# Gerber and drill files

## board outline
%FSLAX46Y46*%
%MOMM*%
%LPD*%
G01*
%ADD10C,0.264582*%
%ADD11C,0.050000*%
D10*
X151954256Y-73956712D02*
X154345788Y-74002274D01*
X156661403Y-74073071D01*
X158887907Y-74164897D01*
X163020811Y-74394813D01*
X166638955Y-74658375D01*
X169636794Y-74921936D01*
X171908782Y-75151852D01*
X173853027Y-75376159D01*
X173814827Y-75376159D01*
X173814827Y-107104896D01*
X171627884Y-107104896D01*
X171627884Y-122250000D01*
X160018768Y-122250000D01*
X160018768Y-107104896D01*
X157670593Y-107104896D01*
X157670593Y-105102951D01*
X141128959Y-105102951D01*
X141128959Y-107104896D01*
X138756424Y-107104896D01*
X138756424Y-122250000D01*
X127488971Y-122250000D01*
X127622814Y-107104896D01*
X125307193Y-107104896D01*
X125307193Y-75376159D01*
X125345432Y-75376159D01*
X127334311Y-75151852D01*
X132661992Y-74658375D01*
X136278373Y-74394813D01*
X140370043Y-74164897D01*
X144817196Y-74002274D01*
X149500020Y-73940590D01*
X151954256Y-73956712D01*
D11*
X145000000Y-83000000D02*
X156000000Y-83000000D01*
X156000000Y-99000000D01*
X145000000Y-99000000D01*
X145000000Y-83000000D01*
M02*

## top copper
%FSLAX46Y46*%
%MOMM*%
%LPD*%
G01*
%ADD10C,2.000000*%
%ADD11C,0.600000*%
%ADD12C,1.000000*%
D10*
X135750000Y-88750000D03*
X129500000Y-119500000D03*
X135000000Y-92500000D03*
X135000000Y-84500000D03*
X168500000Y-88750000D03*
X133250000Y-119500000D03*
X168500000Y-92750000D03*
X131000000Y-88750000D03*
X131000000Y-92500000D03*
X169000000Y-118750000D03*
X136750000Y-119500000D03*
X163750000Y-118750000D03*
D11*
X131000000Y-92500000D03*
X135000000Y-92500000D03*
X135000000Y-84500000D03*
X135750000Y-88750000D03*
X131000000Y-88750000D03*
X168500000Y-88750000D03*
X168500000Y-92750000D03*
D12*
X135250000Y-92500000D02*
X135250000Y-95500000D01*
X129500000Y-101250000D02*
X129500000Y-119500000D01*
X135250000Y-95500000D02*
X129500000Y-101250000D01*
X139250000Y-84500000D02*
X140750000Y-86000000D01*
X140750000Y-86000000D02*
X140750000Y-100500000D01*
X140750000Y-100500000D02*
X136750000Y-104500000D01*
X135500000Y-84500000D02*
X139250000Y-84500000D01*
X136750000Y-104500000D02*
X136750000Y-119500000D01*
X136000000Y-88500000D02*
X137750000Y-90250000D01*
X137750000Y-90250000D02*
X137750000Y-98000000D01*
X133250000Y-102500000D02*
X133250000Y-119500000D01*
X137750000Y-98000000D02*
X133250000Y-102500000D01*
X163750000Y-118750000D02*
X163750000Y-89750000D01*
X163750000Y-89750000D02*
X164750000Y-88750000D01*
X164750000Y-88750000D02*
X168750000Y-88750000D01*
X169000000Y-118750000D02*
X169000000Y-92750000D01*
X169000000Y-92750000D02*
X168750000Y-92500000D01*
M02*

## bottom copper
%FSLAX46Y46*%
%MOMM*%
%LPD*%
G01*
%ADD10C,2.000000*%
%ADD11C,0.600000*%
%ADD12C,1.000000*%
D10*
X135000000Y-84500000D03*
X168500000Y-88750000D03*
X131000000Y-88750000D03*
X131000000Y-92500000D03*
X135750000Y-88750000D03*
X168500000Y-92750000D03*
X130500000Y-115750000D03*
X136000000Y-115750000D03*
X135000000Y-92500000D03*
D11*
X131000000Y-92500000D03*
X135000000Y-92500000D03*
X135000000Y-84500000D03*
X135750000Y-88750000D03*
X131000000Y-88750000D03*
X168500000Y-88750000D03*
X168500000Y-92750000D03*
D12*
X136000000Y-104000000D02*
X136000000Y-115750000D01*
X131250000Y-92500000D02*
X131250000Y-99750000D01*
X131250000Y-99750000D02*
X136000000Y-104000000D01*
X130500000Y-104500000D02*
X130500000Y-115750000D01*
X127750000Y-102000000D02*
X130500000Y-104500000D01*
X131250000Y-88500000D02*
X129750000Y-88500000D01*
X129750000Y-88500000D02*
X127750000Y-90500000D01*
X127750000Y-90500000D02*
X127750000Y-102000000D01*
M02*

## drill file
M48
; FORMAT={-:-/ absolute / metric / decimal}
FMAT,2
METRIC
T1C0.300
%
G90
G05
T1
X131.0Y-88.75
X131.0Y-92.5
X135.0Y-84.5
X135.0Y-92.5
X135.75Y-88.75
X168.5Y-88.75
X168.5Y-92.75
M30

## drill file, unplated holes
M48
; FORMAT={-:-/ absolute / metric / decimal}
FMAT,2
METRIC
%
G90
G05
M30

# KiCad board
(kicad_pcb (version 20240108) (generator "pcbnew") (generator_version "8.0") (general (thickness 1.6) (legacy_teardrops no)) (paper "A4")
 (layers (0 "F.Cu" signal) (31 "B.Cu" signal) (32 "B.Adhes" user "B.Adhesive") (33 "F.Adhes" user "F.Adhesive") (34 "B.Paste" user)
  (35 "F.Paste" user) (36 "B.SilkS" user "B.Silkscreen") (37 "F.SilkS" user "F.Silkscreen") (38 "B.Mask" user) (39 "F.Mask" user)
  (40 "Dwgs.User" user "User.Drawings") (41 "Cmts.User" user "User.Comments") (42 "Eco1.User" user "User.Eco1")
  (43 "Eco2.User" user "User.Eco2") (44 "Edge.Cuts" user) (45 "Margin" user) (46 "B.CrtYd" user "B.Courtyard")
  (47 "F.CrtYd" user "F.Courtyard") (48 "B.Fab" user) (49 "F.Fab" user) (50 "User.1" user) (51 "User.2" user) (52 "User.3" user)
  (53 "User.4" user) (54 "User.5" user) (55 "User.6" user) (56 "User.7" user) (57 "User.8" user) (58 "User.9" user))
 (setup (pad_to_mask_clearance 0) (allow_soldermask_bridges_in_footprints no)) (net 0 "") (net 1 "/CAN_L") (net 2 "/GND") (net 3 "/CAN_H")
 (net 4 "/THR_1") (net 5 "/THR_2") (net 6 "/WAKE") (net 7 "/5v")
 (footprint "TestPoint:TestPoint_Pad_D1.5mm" (layer "F.Cu") (at 135.75 88.75)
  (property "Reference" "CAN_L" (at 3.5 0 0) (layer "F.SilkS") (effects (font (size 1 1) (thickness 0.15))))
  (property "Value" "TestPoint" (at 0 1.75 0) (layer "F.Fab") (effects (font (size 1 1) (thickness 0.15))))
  (pad "1" smd circle (at 0 0) (size 2 2) (layers "F.Cu" "F.Mask") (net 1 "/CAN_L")))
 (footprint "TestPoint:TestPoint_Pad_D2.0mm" (layer "F.Cu") (at 129.5 119.5)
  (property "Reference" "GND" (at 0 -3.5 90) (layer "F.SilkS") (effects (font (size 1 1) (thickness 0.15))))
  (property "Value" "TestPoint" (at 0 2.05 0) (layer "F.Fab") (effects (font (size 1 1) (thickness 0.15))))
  (pad "1" smd circle (at 0 0) (size 2 2) (layers "F.Cu" "F.Mask") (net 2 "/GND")))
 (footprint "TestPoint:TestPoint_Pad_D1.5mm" (layer "F.Cu") (at 135 92.5)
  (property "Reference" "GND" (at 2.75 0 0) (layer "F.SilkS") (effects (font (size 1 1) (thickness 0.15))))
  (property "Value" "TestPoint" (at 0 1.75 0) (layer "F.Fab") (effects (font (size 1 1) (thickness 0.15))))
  (pad "1" smd circle (at 0 0) (size 2 2) (layers "F.Cu" "F.Mask") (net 2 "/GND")))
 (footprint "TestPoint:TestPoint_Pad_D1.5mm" (layer "F.Cu") (at 135 84.5)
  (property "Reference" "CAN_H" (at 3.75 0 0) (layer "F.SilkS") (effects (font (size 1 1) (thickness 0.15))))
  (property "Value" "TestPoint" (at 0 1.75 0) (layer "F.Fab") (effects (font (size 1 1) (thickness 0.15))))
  (pad "1" smd circle (at 0 0) (size 2 2) (layers "F.Cu" "F.Mask") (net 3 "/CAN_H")))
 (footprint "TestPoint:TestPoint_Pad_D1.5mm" (layer "F.Cu") (at 168.5 88.75)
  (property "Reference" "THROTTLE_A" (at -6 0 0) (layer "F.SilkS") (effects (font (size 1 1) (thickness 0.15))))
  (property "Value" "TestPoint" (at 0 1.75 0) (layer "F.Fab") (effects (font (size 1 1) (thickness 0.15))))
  (pad "1" smd circle (at 0 0) (size 2 2) (layers "F.Cu" "F.Mask") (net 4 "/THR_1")))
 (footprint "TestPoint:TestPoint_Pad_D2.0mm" (layer "F.Cu") (at 133.25 119.5)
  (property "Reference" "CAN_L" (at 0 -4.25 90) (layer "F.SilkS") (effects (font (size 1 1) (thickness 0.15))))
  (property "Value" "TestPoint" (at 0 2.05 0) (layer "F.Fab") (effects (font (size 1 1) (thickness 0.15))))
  (pad "1" smd circle (at 0 0) (size 2 2) (layers "F.Cu" "F.Mask") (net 1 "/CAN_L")))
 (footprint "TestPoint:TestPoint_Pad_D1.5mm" (layer "F.Cu") (at 168.5 92.75)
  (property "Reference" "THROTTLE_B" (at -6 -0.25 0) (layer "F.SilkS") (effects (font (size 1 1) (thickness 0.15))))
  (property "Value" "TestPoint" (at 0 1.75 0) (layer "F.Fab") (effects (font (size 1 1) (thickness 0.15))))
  (pad "1" smd circle (at 0 0) (size 2 2) (layers "F.Cu" "F.Mask") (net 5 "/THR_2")))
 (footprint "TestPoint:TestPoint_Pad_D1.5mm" (layer "F.Cu") (at 131 88.75)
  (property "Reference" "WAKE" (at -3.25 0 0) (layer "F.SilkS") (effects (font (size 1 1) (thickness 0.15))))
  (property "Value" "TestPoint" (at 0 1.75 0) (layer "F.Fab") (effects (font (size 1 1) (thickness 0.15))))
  (pad "1" smd circle (at 0 0) (size 2 2) (layers "F.Cu" "F.Mask") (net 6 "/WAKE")))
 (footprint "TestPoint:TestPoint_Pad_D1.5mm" (layer "F.Cu") (at 131 92.5)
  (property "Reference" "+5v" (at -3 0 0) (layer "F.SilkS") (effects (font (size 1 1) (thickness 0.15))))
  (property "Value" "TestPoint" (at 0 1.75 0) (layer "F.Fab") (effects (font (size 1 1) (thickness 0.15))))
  (pad "1" smd circle (at 0 0) (size 2 2) (layers "F.Cu" "F.Mask") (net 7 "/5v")))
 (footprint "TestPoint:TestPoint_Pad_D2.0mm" (layer "F.Cu") (at 169 118.75)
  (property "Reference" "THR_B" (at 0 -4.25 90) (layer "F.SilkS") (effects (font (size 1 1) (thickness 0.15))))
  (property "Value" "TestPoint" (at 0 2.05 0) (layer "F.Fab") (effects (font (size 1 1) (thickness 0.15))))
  (pad "1" smd circle (at 0 0) (size 2 2) (layers "F.Cu" "F.Mask") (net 5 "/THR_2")))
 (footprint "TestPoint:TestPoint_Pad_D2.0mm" (layer "F.Cu") (at 136.75 119.5)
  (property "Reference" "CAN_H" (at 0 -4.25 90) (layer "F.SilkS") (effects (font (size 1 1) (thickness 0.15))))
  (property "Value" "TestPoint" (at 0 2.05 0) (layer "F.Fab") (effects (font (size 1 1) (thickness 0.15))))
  (pad "1" smd circle (at 0 0) (size 2 2) (layers "F.Cu" "F.Mask") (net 3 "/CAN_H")))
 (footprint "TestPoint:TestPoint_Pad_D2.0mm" (layer "F.Cu") (at 163.75 118.75)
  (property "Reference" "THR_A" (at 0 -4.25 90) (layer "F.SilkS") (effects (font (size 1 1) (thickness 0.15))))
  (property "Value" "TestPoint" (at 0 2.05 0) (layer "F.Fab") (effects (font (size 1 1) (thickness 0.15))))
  (pad "1" smd circle (at 0 0) (size 2 2) (layers "F.Cu" "F.Mask") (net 4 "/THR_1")))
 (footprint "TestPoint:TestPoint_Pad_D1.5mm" (layer "B.Cu") (at 135 84.5 180)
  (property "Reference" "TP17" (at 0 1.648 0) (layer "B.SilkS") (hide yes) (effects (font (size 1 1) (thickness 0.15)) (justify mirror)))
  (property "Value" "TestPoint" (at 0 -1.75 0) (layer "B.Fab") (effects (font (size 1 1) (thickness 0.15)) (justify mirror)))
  (pad "1" smd circle (at 0 0 180) (size 2 2) (layers "B.Cu" "B.Mask") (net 3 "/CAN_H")))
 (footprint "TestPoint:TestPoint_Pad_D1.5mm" (layer "B.Cu") (at 168.5 88.75 180)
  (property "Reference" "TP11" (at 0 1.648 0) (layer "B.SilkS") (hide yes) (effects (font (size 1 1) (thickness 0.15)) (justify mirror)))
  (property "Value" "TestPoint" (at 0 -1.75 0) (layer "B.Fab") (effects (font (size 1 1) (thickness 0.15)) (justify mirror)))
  (pad "1" smd circle (at 0 0 180) (size 2 2) (layers "B.Cu" "B.Mask") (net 4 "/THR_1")))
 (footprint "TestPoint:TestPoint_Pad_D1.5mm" (layer "B.Cu") (at 131 88.75 180)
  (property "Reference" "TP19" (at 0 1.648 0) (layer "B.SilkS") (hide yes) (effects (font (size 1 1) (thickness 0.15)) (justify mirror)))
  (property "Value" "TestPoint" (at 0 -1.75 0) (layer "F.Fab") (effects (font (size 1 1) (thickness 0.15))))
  (pad "1" smd circle (at 0 0 180) (size 2 2) (layers "B.Cu" "B.Mask") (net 6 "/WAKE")))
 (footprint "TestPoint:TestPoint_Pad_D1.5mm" (layer "B.Cu") (at 131 92.5 180)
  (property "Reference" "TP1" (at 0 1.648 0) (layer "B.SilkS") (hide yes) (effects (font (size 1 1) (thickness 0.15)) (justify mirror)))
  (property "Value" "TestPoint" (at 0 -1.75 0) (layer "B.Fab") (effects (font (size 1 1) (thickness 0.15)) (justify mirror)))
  (pad "1" smd circle (at 0 0 180) (size 2 2) (layers "B.Cu" "B.Mask") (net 7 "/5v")))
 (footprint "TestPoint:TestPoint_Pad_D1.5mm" (layer "B.Cu") (at 135.75 88.75 180)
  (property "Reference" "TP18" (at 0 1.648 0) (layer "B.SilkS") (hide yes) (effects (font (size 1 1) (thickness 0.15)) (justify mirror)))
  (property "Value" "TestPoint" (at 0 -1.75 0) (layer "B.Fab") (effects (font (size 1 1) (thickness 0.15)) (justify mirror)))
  (pad "1" smd circle (at 0 0 180) (size 2 2) (layers "B.Cu" "B.Mask") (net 1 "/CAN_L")))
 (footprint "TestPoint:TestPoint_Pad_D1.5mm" (layer "B.Cu") (at 168.5 92.75 180)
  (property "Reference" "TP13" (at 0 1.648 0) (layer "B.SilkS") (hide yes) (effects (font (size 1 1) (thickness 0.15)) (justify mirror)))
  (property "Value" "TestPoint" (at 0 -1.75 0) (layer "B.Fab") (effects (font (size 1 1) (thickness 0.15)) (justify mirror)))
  (pad "1" smd circle (at 0 0 180) (size 2 2) (layers "B.Cu" "B.Mask") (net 5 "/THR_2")))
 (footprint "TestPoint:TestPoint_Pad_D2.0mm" (layer "B.Cu") (at 130.5 115.75 180)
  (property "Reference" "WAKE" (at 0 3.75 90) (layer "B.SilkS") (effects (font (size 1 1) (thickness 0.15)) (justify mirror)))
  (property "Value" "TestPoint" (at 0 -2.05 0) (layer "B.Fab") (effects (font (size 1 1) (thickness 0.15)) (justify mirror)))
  (pad "1" smd circle (at 0 0 180) (size 2 2) (layers "B.Cu" "B.Mask") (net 6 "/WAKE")))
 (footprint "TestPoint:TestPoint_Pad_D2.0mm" (layer "B.Cu") (at 136 115.75 180)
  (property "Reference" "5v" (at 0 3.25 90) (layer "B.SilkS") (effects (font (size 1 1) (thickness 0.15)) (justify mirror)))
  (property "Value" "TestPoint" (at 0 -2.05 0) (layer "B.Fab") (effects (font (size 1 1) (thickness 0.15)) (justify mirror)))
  (pad "1" smd circle (at 0 0 180) (size 2 2) (layers "B.Cu" "B.Mask") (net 7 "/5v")))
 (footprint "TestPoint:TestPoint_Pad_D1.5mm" (layer "B.Cu") (at 135 92.5 180)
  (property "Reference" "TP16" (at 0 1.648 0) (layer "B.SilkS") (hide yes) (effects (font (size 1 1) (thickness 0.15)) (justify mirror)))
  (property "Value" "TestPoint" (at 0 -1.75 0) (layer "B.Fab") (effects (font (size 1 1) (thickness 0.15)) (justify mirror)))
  (pad "1" smd circle (at 0 0 180) (size 2 2) (layers "B.Cu" "B.Mask") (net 2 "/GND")))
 (gr_poly
  (pts (xy 151.954256 73.956712) (xy 154.345788 74.002274) (xy 156.661403 74.073071) (xy 158.887907 74.164897) (xy 163.020811 74.394813)
   (xy 166.638955 74.658375) (xy 169.636794 74.921936) (xy 171.908782 75.151852) (xy 173.853027 75.376159) (xy 173.814827 75.376159)
   (xy 173.814827 107.104896) (xy 171.627884 107.104896) (xy 171.627884 122.25) (xy 160.018768 122.25) (xy 160.018768 107.104896)
   (xy 157.670593 107.104896) (xy 157.670593 105.102951) (xy 141.128959 105.102951) (xy 141.128959 107.104896) (xy 138.756424 107.104896)
   (xy 138.756424 122.25) (xy 127.488971 122.25) (xy 127.622814 107.104896) (xy 125.307193 107.104896) (xy 125.307193 75.376159)
   (xy 125.345432 75.376159) (xy 127.334311 75.151852) (xy 132.661992 74.658375) (xy 136.278373 74.394813) (xy 140.370043 74.164897)
   (xy 144.817196 74.002274) (xy 149.50002 73.94059))
  (stroke (width 0.264582) (type solid)) (fill none) (layer "Edge.Cuts"))
 (gr_rect (start 145 83) (end 156 99) (stroke (width 0.05) (type default)) (fill none) (layer "Edge.Cuts"))
 (gr_poly
  (pts (xy 149.50002 73.94059) (xy 149.5 73.94059) (xy 149.50003 73.94059)) (stroke (width 0.264582) (type solid)) (fill none)
  (layer "Edge.Cuts"))
 (via (at 131 92.5) (size 0.6) (drill 0.3) (layers "F.Cu" "B.Cu") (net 7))
 (segment (start 136 104) (end 136 115.75) (width 1) (layer "B.Cu") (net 7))
 (segment (start 131.25 92.5) (end 131.25 99.75) (width 1) (layer "B.Cu") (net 7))
 (segment (start 131.25 99.75) (end 136 104) (width 1) (layer "B.Cu") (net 7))
 (segment (start 135.25 92.5) (end 135.25 95.5) (width 1) (layer "F.Cu") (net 2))
 (segment (start 129.5 101.25) (end 129.5 119.5) (width 1) (layer "F.Cu") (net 2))
 (segment (start 135.25 95.5) (end 129.5 101.25) (width 1) (layer "F.Cu") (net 2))
 (via (at 135 92.5) (size 0.6) (drill 0.3) (layers "F.Cu" "B.Cu") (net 2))
 (segment (start 139.25 84.5) (end 140.75 86) (width 1) (layer "F.Cu") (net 3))
 (segment (start 140.75 86) (end 140.75 100.5) (width 1) (layer "F.Cu") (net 3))
 (segment (start 140.75 100.5) (end 136.75 104.5) (width 1) (layer "F.Cu") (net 3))
 (segment (start 135.5 84.5) (end 139.25 84.5) (width 1) (layer "F.Cu") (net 3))
 (segment (start 136.75 104.5) (end 136.75 119.5) (width 1) (layer "F.Cu") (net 3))
 (via (at 135 84.5) (size 0.6) (drill 0.3) (layers "F.Cu" "B.Cu") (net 3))
 (segment (start 136 88.5) (end 137.75 90.25) (width 1) (layer "F.Cu") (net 1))
 (segment (start 137.75 90.25) (end 137.75 98) (width 1) (layer "F.Cu") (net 1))
 (segment (start 133.25 102.5) (end 133.25 119.5) (width 1) (layer "F.Cu") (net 1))
 (segment (start 137.75 98) (end 133.25 102.5) (width 1) (layer "F.Cu") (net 1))
 (via (at 135.75 88.75) (size 0.6) (drill 0.3) (layers "F.Cu" "B.Cu") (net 1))
 (via (at 131 88.75) (size 0.6) (drill 0.3) (layers "F.Cu" "B.Cu") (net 6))
 (segment (start 130.5 104.5) (end 130.5 115.75) (width 1) (layer "B.Cu") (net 6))
 (segment (start 127.75 102) (end 130.5 104.5) (width 1) (layer "B.Cu") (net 6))
 (segment (start 131.25 88.5) (end 129.75 88.5) (width 1) (layer "B.Cu") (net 6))
 (segment (start 129.75 88.5) (end 127.75 90.5) (width 1) (layer "B.Cu") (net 6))
 (segment (start 127.75 90.5) (end 127.75 102) (width 1) (layer "B.Cu") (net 6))
 (segment (start 163.75 118.75) (end 163.75 89.75) (width 1) (layer "F.Cu") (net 4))
 (segment (start 163.75 89.75) (end 164.75 88.75) (width 1) (layer "F.Cu") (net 4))
 (segment (start 164.75 88.75) (end 168.75 88.75) (width 1) (layer "F.Cu") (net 4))
 (via (at 168.5 88.75) (size 0.6) (drill 0.3) (layers "F.Cu" "B.Cu") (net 4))
 (segment (start 169 118.75) (end 169 92.75) (width 1) (layer "F.Cu") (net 5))
 (segment (start 169 92.75) (end 168.75 92.5) (width 1) (layer "F.Cu") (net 5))
 (via (at 168.5 92.75) (size 0.6) (drill 0.3) (layers "F.Cu" "B.Cu") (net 5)))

